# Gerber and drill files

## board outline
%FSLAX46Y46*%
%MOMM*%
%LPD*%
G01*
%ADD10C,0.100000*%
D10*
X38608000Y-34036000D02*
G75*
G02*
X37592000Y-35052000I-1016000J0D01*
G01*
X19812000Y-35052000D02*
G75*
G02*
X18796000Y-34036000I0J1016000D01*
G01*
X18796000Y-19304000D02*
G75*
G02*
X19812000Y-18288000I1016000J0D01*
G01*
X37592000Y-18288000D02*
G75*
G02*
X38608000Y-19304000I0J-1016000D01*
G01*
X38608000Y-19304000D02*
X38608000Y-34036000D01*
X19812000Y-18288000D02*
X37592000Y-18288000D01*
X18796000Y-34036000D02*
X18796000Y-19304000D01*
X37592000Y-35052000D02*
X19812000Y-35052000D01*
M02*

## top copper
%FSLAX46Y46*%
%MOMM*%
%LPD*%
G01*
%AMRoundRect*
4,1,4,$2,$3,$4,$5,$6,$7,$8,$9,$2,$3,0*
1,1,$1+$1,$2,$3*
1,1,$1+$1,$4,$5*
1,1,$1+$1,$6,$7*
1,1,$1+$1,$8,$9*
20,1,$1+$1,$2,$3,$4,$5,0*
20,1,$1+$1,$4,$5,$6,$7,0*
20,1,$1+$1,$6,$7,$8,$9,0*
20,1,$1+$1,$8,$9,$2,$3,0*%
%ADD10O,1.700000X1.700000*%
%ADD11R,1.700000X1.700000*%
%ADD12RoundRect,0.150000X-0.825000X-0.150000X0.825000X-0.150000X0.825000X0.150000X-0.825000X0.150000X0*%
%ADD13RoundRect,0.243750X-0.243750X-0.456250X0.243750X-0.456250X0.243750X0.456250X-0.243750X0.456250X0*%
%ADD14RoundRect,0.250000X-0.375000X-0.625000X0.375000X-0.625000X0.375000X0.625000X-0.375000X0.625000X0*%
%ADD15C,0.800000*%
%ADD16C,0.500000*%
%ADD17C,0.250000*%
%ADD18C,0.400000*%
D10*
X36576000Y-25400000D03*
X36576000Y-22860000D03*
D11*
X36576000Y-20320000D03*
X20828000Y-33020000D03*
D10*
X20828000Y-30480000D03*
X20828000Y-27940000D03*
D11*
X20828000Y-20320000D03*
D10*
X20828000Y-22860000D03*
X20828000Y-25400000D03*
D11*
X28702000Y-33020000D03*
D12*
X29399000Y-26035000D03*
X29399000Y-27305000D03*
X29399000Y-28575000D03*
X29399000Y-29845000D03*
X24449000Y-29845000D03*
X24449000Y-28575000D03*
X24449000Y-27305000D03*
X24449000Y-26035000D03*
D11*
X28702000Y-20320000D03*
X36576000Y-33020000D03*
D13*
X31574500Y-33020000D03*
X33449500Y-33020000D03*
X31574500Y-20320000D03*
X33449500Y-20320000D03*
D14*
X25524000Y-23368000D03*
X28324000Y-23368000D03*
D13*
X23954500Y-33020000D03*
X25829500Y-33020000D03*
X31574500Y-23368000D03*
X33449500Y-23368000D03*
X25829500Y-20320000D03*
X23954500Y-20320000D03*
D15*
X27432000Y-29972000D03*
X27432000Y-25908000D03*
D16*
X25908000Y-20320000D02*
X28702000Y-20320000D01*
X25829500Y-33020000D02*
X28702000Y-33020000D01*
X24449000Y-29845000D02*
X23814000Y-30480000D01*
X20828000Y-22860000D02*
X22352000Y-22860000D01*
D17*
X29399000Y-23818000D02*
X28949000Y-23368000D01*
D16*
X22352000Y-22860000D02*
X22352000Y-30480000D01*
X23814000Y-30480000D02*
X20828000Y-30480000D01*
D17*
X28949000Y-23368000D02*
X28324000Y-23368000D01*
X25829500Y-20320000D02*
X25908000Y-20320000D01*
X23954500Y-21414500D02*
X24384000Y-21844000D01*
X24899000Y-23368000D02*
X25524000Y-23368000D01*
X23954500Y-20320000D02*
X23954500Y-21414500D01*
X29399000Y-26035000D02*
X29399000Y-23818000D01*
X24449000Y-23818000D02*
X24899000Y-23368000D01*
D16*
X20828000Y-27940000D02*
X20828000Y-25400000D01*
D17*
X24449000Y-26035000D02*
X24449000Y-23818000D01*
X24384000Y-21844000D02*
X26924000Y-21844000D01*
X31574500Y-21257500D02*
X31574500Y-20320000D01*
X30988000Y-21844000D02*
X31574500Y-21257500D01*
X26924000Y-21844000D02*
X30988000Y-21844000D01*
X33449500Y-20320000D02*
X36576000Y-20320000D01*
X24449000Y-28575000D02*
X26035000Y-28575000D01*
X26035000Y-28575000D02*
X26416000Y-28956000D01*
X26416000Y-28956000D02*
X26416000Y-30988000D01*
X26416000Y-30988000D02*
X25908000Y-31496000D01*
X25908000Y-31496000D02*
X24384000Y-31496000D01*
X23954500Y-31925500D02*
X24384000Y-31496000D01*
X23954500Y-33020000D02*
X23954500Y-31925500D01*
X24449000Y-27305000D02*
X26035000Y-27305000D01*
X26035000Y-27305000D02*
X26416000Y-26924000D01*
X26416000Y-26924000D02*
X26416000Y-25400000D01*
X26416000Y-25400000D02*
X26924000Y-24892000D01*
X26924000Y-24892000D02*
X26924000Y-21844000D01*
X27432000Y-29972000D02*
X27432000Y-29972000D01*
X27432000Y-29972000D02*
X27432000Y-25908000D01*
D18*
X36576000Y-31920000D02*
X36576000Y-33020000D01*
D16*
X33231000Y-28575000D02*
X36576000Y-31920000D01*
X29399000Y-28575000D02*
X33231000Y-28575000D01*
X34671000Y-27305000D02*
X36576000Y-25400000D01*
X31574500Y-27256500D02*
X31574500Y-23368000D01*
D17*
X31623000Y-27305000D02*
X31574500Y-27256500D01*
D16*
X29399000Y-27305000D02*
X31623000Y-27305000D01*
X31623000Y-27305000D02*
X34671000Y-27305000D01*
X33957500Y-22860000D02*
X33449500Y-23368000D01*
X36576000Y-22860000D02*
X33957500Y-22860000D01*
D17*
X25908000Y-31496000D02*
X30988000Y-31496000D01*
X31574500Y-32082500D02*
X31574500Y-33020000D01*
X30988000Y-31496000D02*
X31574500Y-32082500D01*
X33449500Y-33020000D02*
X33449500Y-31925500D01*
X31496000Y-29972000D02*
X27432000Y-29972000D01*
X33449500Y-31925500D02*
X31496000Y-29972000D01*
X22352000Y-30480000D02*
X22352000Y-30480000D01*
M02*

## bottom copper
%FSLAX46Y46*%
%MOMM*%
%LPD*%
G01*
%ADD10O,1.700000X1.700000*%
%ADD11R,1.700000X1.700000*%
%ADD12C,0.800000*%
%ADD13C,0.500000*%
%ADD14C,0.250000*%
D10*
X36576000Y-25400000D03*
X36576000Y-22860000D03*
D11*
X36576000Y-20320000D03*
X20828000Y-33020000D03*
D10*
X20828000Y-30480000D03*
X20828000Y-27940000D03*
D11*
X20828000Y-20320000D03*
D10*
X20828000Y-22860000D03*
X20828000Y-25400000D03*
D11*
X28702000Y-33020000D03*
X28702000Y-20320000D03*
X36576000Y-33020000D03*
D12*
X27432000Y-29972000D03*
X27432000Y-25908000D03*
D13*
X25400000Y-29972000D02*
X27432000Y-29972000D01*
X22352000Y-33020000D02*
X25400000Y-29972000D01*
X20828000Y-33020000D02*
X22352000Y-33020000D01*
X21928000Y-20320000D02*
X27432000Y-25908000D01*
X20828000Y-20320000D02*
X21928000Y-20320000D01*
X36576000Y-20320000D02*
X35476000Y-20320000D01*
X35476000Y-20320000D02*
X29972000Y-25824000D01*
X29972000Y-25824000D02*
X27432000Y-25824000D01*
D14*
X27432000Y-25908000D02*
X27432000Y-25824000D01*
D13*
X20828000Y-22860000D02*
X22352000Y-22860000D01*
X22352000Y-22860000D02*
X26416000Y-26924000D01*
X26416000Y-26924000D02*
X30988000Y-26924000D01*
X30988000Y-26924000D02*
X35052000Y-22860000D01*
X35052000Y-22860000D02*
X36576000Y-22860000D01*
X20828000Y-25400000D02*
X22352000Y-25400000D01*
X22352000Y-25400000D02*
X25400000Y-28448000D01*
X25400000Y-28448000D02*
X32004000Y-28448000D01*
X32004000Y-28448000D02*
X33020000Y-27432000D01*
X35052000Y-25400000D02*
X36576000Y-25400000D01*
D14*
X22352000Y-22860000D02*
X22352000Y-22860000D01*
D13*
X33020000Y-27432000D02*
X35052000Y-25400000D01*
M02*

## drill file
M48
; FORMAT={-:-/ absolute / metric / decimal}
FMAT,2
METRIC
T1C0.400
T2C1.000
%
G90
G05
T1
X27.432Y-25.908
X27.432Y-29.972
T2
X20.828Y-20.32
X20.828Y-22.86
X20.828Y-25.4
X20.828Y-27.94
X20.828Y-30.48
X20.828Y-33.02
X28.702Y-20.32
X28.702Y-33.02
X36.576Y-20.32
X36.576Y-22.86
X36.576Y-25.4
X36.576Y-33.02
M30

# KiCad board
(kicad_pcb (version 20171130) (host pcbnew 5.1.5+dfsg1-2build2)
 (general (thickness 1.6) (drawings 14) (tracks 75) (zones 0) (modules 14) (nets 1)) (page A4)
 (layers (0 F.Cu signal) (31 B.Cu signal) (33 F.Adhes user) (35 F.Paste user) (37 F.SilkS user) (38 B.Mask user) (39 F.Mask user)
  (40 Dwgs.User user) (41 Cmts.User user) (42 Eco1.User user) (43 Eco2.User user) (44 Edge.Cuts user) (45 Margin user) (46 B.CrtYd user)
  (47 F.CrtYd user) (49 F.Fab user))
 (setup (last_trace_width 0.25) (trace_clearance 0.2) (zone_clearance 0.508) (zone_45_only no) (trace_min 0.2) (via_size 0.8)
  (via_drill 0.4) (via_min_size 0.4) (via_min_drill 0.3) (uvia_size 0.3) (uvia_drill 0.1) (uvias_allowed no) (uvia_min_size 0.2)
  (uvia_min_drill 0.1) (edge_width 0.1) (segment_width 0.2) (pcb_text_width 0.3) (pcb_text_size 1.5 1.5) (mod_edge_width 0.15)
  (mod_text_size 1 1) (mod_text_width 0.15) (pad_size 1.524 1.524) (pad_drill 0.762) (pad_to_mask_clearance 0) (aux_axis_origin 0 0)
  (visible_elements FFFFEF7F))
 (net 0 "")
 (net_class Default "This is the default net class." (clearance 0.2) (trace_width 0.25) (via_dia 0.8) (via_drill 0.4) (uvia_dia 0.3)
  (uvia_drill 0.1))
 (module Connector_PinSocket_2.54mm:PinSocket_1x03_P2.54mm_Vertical (layer F.Cu) (at 36.576 20.32)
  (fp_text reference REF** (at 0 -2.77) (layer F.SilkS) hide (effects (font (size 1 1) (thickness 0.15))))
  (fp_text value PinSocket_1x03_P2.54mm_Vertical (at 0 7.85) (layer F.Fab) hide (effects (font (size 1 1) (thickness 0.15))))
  (pad 3 thru_hole oval (at 0 5.08) (size 1.7 1.7) (drill 1) (layers *.Cu *.Mask))
  (pad 2 thru_hole oval (at 0 2.54) (size 1.7 1.7) (drill 1) (layers *.Cu *.Mask))
  (pad 1 thru_hole rect (at 0 0) (size 1.7 1.7) (drill 1) (layers *.Cu *.Mask)))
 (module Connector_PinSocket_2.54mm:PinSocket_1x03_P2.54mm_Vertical (layer F.Cu) (at 20.828 33.02 180)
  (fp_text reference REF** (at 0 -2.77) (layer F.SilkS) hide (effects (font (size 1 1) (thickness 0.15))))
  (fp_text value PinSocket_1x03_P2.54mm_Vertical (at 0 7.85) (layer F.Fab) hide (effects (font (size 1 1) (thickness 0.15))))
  (pad 1 thru_hole rect (at 0 0 180) (size 1.7 1.7) (drill 1) (layers *.Cu *.Mask))
  (pad 2 thru_hole oval (at 0 2.54 180) (size 1.7 1.7) (drill 1) (layers *.Cu *.Mask))
  (pad 3 thru_hole oval (at 0 5.08 180) (size 1.7 1.7) (drill 1) (layers *.Cu *.Mask)))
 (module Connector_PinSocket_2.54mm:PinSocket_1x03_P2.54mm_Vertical (layer F.Cu) (at 20.828 20.32)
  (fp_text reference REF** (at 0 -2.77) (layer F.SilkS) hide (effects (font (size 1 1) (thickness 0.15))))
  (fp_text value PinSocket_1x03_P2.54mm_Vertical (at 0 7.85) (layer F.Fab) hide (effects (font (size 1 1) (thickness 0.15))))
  (pad 1 thru_hole rect (at 0 0) (size 1.7 1.7) (drill 1) (layers *.Cu *.Mask))
  (pad 2 thru_hole oval (at 0 2.54) (size 1.7 1.7) (drill 1) (layers *.Cu *.Mask))
  (pad 3 thru_hole oval (at 0 5.08) (size 1.7 1.7) (drill 1) (layers *.Cu *.Mask)))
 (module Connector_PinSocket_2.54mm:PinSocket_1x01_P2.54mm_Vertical (layer F.Cu) (at 28.702 33.02)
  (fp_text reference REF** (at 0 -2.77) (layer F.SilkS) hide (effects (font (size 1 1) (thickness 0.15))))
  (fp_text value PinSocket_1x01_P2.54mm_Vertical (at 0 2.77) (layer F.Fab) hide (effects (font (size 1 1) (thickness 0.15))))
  (pad 1 thru_hole rect (at 0 0) (size 1.7 1.7) (drill 1) (layers *.Cu *.Mask)))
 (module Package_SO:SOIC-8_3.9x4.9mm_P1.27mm (layer F.Cu) (at 26.924 27.94)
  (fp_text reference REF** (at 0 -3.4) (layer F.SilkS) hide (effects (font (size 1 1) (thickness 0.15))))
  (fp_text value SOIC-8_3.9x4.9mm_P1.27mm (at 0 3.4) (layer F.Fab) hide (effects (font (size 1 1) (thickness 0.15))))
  (pad 8 smd roundrect (at 2.475 -1.905) (size 1.95 0.6) (layers F.Cu F.Paste F.Mask) (roundrect_rratio 0.25))
  (pad 7 smd roundrect (at 2.475 -0.635) (size 1.95 0.6) (layers F.Cu F.Paste F.Mask) (roundrect_rratio 0.25))
  (pad 6 smd roundrect (at 2.475 0.635) (size 1.95 0.6) (layers F.Cu F.Paste F.Mask) (roundrect_rratio 0.25))
  (pad 5 smd roundrect (at 2.475 1.905) (size 1.95 0.6) (layers F.Cu F.Paste F.Mask) (roundrect_rratio 0.25))
  (pad 4 smd roundrect (at -2.475 1.905) (size 1.95 0.6) (layers F.Cu F.Paste F.Mask) (roundrect_rratio 0.25))
  (pad 3 smd roundrect (at -2.475 0.635) (size 1.95 0.6) (layers F.Cu F.Paste F.Mask) (roundrect_rratio 0.25))
  (pad 2 smd roundrect (at -2.475 -0.635) (size 1.95 0.6) (layers F.Cu F.Paste F.Mask) (roundrect_rratio 0.25))
  (pad 1 smd roundrect (at -2.475 -1.905) (size 1.95 0.6) (layers F.Cu F.Paste F.Mask) (roundrect_rratio 0.25)))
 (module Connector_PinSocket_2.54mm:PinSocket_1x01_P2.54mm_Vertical (layer F.Cu) (at 28.702 20.32 180)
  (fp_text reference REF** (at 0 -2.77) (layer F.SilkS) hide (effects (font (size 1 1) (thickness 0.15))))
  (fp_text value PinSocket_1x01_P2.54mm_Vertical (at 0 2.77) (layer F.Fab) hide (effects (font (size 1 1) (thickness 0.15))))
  (pad 1 thru_hole rect (at 0 0 180) (size 1.7 1.7) (drill 1) (layers *.Cu *.Mask)))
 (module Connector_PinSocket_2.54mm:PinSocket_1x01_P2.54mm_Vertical (layer F.Cu) (at 36.576 33.02)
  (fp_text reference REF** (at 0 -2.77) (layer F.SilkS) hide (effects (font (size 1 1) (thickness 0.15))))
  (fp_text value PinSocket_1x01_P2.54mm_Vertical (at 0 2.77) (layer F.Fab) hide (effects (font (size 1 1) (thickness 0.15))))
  (pad 1 thru_hole rect (at 0 0) (size 1.7 1.7) (drill 1) (layers *.Cu *.Mask)))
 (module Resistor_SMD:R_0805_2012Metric (layer F.Cu) (at 32.512 33.02)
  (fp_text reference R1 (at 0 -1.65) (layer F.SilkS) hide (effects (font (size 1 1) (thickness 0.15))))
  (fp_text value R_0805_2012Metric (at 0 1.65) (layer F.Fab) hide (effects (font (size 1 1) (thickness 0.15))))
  (pad 1 smd roundrect (at -0.9375 0) (size 0.975 1.4) (layers F.Cu F.Paste F.Mask) (roundrect_rratio 0.25))
  (pad 2 smd roundrect (at 0.9375 0) (size 0.975 1.4) (layers F.Cu F.Paste F.Mask) (roundrect_rratio 0.25)))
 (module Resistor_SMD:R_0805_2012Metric (layer F.Cu) (at 32.512 20.32)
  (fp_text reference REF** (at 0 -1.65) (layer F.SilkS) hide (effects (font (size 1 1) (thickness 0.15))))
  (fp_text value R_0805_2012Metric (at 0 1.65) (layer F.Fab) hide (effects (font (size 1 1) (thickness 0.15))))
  (pad 1 smd roundrect (at -0.9375 0) (size 0.975 1.4) (layers F.Cu F.Paste F.Mask) (roundrect_rratio 0.25))
  (pad 2 smd roundrect (at 0.9375 0) (size 0.975 1.4) (layers F.Cu F.Paste F.Mask) (roundrect_rratio 0.25)))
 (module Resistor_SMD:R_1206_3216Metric (layer F.Cu) (at 26.924 23.368)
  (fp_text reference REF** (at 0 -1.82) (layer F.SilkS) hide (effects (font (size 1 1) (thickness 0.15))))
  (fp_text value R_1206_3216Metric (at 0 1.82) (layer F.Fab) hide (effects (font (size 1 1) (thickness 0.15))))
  (pad 1 smd roundrect (at -1.4 0) (size 1.25 1.75) (layers F.Cu F.Paste F.Mask) (roundrect_rratio 0.2))
  (pad 2 smd roundrect (at 1.4 0) (size 1.25 1.75) (layers F.Cu F.Paste F.Mask) (roundrect_rratio 0.2)))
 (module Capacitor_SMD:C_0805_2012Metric (layer F.Cu) (at 24.892 33.02)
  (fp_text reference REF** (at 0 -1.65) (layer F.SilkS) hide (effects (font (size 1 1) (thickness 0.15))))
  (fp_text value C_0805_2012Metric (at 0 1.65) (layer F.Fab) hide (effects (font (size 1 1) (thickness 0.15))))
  (pad 1 smd roundrect (at -0.9375 0) (size 0.975 1.4) (layers F.Cu F.Paste F.Mask) (roundrect_rratio 0.25))
  (pad 2 smd roundrect (at 0.9375 0) (size 0.975 1.4) (layers F.Cu F.Paste F.Mask) (roundrect_rratio 0.25)))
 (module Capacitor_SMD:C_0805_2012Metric (layer F.Cu) (at 32.512 23.368)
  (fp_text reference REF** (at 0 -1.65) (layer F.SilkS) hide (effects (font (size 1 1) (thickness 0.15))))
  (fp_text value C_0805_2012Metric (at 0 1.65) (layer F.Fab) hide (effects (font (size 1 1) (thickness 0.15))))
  (pad 1 smd roundrect (at -0.9375 0) (size 0.975 1.4) (layers F.Cu F.Paste F.Mask) (roundrect_rratio 0.25))
  (pad 2 smd roundrect (at 0.9375 0) (size 0.975 1.4) (layers F.Cu F.Paste F.Mask) (roundrect_rratio 0.25)))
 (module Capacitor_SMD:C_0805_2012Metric (layer F.Cu) (at 24.892 20.32)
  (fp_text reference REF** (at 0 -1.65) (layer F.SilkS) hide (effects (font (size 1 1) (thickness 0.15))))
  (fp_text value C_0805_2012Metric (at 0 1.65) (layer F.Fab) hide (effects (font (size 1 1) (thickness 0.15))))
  (pad 2 smd roundrect (at 0.9375 0) (size 0.975 1.4) (layers F.Cu F.Paste F.Mask) (roundrect_rratio 0.25))
  (pad 1 smd roundrect (at -0.9375 0) (size 0.975 1.4) (layers F.Cu F.Paste F.Mask) (roundrect_rratio 0.25)))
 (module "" (layer F.Cu) (at 33.02 36.83)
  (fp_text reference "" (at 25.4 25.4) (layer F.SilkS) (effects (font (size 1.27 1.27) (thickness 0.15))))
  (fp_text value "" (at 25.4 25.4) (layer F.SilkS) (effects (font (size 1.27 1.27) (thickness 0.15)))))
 (gr_arc (start 37.592 34.036) (end 37.592 35.052) (angle -90) (layer Edge.Cuts) (width 0.1))
 (gr_arc (start 19.812 34.036) (end 18.796 34.036) (angle -90) (layer Edge.Cuts) (width 0.1))
 (gr_arc (start 19.812 19.304) (end 19.812 18.288) (angle -90) (layer Edge.Cuts) (width 0.1))
 (gr_arc (start 37.592 19.304) (end 38.608 19.304) (angle -90) (layer Edge.Cuts) (width 0.1))
 (gr_line (start 38.608 19.304) (end 38.608 34.036) (layer Edge.Cuts) (width 0.1))
 (gr_line (start 19.812 18.288) (end 37.592 18.288) (layer Edge.Cuts) (width 0.1))
 (gr_line (start 18.796 34.036) (end 18.796 19.304) (layer Edge.Cuts) (width 0.1))
 (gr_line (start 37.592 35.052) (end 19.812 35.052) (layer Edge.Cuts) (width 0.1))
 (segment (start 25.908 20.32) (end 28.702 20.32) (width 0.5) (layer F.Cu) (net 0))
 (segment (start 25.8295 33.02) (end 28.702 33.02) (width 0.5) (layer F.Cu) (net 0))
 (segment (start 24.449 29.845) (end 23.814 30.48) (width 0.5) (layer F.Cu) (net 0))
 (segment (start 20.828 22.86) (end 22.352 22.86) (width 0.5) (layer F.Cu) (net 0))
 (segment (start 29.399 23.818) (end 28.949 23.368) (width 0.25) (layer F.Cu) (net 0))
 (segment (start 22.352 22.86) (end 22.352 30.48) (width 0.5) (layer F.Cu) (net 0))
 (segment (start 23.814 30.48) (end 20.828 30.48) (width 0.5) (layer F.Cu) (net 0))
 (segment (start 28.949 23.368) (end 28.324 23.368) (width 0.25) (layer F.Cu) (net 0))
 (segment (start 25.8295 20.32) (end 25.908 20.32) (width 0.25) (layer F.Cu) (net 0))
 (segment (start 23.9545 21.4145) (end 24.384 21.844) (width 0.25) (layer F.Cu) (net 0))
 (segment (start 24.899 23.368) (end 25.524 23.368) (width 0.25) (layer F.Cu) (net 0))
 (segment (start 23.9545 20.32) (end 23.9545 21.4145) (width 0.25) (layer F.Cu) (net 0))
 (segment (start 29.399 26.035) (end 29.399 23.818) (width 0.25) (layer F.Cu) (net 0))
 (segment (start 24.449 23.818) (end 24.899 23.368) (width 0.25) (layer F.Cu) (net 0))
 (segment (start 20.828 27.94) (end 20.828 25.4) (width 0.5) (layer F.Cu) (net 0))
 (segment (start 24.449 26.035) (end 24.449 23.818) (width 0.25) (layer F.Cu) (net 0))
 (segment (start 24.384 21.844) (end 26.924 21.844) (width 0.25) (layer F.Cu) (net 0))
 (segment (start 31.5745 21.2575) (end 31.5745 20.32) (width 0.25) (layer F.Cu) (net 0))
 (segment (start 30.988 21.844) (end 31.5745 21.2575) (width 0.25) (layer F.Cu) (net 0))
 (segment (start 26.924 21.844) (end 30.988 21.844) (width 0.25) (layer F.Cu) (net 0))
 (segment (start 33.4495 20.32) (end 36.576 20.32) (width 0.25) (layer F.Cu) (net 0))
 (segment (start 24.449 28.575) (end 26.035 28.575) (width 0.25) (layer F.Cu) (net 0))
 (segment (start 26.035 28.575) (end 26.416 28.956) (width 0.25) (layer F.Cu) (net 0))
 (segment (start 26.416 28.956) (end 26.416 30.988) (width 0.25) (layer F.Cu) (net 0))
 (segment (start 26.416 30.988) (end 25.908 31.496) (width 0.25) (layer F.Cu) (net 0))
 (segment (start 25.908 31.496) (end 24.384 31.496) (width 0.25) (layer F.Cu) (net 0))
 (segment (start 23.9545 31.9255) (end 24.384 31.496) (width 0.25) (layer F.Cu) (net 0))
 (segment (start 23.9545 33.02) (end 23.9545 31.9255) (width 0.25) (layer F.Cu) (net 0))
 (segment (start 24.449 27.305) (end 26.035 27.305) (width 0.25) (layer F.Cu) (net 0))
 (segment (start 26.035 27.305) (end 26.416 26.924) (width 0.25) (layer F.Cu) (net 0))
 (segment (start 26.416 26.924) (end 26.416 25.4) (width 0.25) (layer F.Cu) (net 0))
 (segment (start 26.416 25.4) (end 26.924 24.892) (width 0.25) (layer F.Cu) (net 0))
 (segment (start 26.924 24.892) (end 26.924 21.844) (width 0.25) (layer F.Cu) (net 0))
 (segment (start 27.432 29.972) (end 27.432 29.972) (width 0.25) (layer F.Cu) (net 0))
 (via (at 27.432 29.972) (size 0.8) (drill 0.4) (layers F.Cu B.Cu) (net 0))
 (segment (start 25.4 29.972) (end 27.432 29.972) (width 0.5) (layer B.Cu) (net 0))
 (segment (start 22.352 33.02) (end 25.4 29.972) (width 0.5) (layer B.Cu) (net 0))
 (segment (start 20.828 33.02) (end 22.352 33.02) (width 0.5) (layer B.Cu) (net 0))
 (segment (start 21.928 20.32) (end 27.432 25.908) (width 0.5) (layer B.Cu) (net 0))
 (segment (start 20.828 20.32) (end 21.928 20.32) (width 0.5) (layer B.Cu) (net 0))
 (segment (start 36.576 20.32) (end 35.476 20.32) (width 0.5) (layer B.Cu) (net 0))
 (segment (start 35.476 20.32) (end 29.972 25.824) (width 0.5) (layer B.Cu) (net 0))
 (segment (start 29.972 25.824) (end 27.432 25.824) (width 0.5) (layer B.Cu) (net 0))
 (segment (start 27.432 25.908) (end 27.432 25.824) (width 0.25) (layer B.Cu) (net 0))
 (via (at 27.432 25.908) (size 0.8) (drill 0.4) (layers F.Cu B.Cu) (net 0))
 (segment (start 27.432 29.972) (end 27.432 25.908) (width 0.25) (layer F.Cu) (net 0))
 (segment (start 36.576 31.92) (end 36.576 33.02) (width 0.4) (layer F.Cu) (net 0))
 (segment (start 33.231 28.575) (end 36.576 31.92) (width 0.5) (layer F.Cu) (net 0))
 (segment (start 29.399 28.575) (end 33.231 28.575) (width 0.5) (layer F.Cu) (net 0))
 (segment (start 20.828 22.86) (end 22.352 22.86) (width 0.5) (layer B.Cu) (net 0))
 (segment (start 22.352 22.86) (end 26.416 26.924) (width 0.5) (layer B.Cu) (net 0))
 (segment (start 26.416 26.924) (end 30.988 26.924) (width 0.5) (layer B.Cu) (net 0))
 (segment (start 30.988 26.924) (end 35.052 22.86) (width 0.5) (layer B.Cu) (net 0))
 (segment (start 35.052 22.86) (end 36.576 22.86) (width 0.5) (layer B.Cu) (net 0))
 (segment (start 20.828 25.4) (end 22.352 25.4) (width 0.5) (layer B.Cu) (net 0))
 (segment (start 22.352 25.4) (end 25.4 28.448) (width 0.5) (layer B.Cu) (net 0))
 (segment (start 25.4 28.448) (end 32.004 28.448) (width 0.5) (layer B.Cu) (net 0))
 (segment (start 32.004 28.448) (end 33.02 27.432) (width 0.5) (layer B.Cu) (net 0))
 (segment (start 35.052 25.4) (end 36.576 25.4) (width 0.5) (layer B.Cu) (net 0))
 (segment (start 34.671 27.305) (end 36.576 25.4) (width 0.5) (layer F.Cu) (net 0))
 (segment (start 31.5745 27.2565) (end 31.5745 23.368) (width 0.5) (layer F.Cu) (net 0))
 (segment (start 31.623 27.305) (end 31.5745 27.2565) (width 0.25) (layer F.Cu) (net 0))
 (segment (start 29.399 27.305) (end 31.623 27.305) (width 0.5) (layer F.Cu) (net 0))
 (segment (start 31.623 27.305) (end 34.671 27.305) (width 0.5) (layer F.Cu) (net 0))
 (segment (start 33.9575 22.86) (end 33.4495 23.368) (width 0.5) (layer F.Cu) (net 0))
 (segment (start 36.576 22.86) (end 33.9575 22.86) (width 0.5) (layer F.Cu) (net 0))
 (segment (start 25.908 31.496) (end 30.988 31.496) (width 0.25) (layer F.Cu) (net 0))
 (segment (start 31.5745 32.0825) (end 31.5745 33.02) (width 0.25) (layer F.Cu) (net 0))
 (segment (start 30.988 31.496) (end 31.5745 32.0825) (width 0.25) (layer F.Cu) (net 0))
 (segment (start 33.4495 33.02) (end 33.4495 31.9255) (width 0.25) (layer F.Cu) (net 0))
 (segment (start 31.496 29.972) (end 27.432 29.972) (width 0.25) (layer F.Cu) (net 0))
 (segment (start 33.4495 31.9255) (end 31.496 29.972) (width 0.25) (layer F.Cu) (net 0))
 (segment (start 22.352 22.86) (end 22.352 22.86) (width 0.25) (layer B.Cu) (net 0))
 (segment (start 33.02 27.432) (end 35.052 25.4) (width 0.5) (layer B.Cu) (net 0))
 (segment (start 22.352 30.48) (end 22.352 30.48) (width 0.25) (layer F.Cu) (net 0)))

